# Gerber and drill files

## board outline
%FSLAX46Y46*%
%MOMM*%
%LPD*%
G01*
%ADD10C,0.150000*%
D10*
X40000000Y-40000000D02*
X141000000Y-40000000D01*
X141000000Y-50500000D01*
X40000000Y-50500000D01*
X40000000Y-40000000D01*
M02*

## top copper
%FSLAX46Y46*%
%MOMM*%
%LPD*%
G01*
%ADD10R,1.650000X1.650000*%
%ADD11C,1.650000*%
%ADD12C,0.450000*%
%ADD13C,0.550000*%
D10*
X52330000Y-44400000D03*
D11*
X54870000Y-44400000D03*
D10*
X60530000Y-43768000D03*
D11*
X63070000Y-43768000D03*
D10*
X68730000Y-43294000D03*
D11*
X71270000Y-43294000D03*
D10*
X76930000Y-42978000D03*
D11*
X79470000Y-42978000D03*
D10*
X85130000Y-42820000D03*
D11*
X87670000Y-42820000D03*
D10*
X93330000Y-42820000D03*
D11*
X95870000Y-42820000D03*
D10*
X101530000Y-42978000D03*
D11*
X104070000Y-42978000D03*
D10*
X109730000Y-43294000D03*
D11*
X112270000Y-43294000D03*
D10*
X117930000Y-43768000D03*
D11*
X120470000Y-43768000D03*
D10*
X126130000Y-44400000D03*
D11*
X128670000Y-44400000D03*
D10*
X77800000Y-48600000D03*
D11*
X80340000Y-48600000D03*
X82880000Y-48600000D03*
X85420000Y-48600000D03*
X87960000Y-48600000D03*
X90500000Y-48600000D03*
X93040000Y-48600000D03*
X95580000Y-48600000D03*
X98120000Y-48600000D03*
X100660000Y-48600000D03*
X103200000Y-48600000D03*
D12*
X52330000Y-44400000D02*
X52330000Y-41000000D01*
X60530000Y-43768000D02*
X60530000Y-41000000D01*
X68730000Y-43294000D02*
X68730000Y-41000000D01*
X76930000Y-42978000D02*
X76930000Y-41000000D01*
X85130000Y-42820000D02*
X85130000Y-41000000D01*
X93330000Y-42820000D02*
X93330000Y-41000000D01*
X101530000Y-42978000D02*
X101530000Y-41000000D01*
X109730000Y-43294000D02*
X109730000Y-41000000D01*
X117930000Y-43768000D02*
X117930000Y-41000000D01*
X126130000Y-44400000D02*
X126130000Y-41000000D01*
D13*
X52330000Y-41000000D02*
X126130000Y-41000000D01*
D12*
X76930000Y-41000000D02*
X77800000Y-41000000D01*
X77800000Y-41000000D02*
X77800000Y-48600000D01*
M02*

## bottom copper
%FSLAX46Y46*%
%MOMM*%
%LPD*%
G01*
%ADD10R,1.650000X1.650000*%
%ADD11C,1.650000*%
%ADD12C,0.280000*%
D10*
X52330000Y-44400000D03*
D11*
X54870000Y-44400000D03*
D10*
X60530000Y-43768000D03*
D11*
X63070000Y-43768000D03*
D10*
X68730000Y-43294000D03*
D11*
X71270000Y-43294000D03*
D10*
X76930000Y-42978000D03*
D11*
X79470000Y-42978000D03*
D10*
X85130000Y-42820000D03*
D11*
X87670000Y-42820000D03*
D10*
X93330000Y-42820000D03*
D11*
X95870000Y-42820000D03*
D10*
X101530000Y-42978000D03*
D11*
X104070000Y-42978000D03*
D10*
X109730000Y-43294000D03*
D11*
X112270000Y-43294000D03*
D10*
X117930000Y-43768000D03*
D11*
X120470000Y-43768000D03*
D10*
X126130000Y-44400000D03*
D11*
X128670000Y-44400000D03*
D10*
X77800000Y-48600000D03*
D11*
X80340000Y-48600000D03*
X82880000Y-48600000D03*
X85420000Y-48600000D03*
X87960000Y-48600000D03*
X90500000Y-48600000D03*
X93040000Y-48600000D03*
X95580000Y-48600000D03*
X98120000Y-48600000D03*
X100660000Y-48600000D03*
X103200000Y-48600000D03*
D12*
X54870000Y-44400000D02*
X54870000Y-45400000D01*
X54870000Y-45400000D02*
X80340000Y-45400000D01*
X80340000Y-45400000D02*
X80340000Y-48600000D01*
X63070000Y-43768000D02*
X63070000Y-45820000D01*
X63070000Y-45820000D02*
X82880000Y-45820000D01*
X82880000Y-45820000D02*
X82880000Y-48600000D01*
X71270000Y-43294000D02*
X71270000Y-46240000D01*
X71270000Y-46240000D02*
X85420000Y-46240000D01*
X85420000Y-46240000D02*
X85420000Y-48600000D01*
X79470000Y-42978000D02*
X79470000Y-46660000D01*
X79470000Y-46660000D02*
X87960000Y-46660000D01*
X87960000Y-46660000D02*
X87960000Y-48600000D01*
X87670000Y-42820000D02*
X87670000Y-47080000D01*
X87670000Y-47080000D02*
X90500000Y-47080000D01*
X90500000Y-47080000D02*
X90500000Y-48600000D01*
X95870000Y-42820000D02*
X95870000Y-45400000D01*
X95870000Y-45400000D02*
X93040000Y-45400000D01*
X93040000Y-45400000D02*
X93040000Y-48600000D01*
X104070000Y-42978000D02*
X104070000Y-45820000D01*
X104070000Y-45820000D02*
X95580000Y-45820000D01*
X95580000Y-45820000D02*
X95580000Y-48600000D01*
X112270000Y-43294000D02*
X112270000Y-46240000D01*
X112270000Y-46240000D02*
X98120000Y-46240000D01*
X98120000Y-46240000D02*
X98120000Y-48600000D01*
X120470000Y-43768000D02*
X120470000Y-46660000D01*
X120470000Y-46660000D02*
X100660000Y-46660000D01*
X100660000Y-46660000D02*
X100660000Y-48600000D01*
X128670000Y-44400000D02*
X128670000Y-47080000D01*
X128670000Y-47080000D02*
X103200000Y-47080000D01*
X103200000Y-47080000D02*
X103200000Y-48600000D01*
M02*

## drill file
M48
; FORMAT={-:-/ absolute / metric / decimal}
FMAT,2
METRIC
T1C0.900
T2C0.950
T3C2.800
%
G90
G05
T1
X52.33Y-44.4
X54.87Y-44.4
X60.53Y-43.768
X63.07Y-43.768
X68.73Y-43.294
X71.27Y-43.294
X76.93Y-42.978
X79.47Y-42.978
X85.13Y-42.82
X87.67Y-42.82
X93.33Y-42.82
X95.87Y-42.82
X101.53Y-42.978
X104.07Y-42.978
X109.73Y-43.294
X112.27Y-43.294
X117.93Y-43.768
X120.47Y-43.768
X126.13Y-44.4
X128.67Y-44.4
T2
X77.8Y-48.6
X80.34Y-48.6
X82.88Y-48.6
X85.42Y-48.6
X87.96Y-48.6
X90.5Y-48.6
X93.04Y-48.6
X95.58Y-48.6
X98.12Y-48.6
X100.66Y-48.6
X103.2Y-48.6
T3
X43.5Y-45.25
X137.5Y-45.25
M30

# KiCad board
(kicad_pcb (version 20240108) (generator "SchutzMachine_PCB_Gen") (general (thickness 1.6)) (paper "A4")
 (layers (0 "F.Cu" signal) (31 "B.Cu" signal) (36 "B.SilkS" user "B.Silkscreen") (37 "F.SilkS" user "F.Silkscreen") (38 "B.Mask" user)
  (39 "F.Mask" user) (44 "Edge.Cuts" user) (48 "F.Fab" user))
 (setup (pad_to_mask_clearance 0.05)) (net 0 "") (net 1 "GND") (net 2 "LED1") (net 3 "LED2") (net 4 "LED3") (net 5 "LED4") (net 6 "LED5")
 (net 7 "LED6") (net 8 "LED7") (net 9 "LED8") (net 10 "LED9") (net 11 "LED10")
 (gr_rect (start 40.0 40.0) (end 141.0 50.5) (stroke (width 0.15) (type solid)) (fill none) (layer "Edge.Cuts"))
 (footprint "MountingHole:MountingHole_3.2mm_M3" (layer "F.Cu") (at 43.5 45.25)
  (pad "" np_thru_hole circle (at 0 0) (size 2.8 2.8) (drill 2.8) (layers "*.Cu" "*.Mask")))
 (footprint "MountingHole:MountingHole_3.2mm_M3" (layer "F.Cu") (at 137.5 45.25)
  (pad "" np_thru_hole circle (at 0 0) (size 2.8 2.8) (drill 2.8) (layers "*.Cu" "*.Mask")))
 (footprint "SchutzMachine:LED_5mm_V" (layer "F.Cu") (at 53.6 44.4 0)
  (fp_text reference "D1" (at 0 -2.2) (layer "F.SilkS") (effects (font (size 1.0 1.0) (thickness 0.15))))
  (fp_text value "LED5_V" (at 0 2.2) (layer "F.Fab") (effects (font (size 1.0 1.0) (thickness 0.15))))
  (pad "1" thru_hole rect (at -1.27 0.0) (size 1.65 1.65) (drill 0.9) (layers "*.Cu" "*.Mask") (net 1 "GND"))
  (pad "2" thru_hole circle (at 1.27 0.0) (size 1.65 1.65) (drill 0.9) (layers "*.Cu" "*.Mask") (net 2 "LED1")))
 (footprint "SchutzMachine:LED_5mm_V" (layer "F.Cu") (at 61.8 43.768 0)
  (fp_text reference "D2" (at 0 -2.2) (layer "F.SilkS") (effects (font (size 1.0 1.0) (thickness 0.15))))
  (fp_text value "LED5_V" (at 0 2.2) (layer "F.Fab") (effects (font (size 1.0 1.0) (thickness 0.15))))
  (pad "1" thru_hole rect (at -1.27 0.0) (size 1.65 1.65) (drill 0.9) (layers "*.Cu" "*.Mask") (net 1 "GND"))
  (pad "2" thru_hole circle (at 1.27 0.0) (size 1.65 1.65) (drill 0.9) (layers "*.Cu" "*.Mask") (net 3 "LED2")))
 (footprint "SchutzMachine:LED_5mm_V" (layer "F.Cu") (at 70.0 43.294 0)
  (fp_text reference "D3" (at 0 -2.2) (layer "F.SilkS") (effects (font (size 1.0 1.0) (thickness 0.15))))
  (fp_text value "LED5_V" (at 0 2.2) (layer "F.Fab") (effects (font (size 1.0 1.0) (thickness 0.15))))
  (pad "1" thru_hole rect (at -1.27 0.0) (size 1.65 1.65) (drill 0.9) (layers "*.Cu" "*.Mask") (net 1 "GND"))
  (pad "2" thru_hole circle (at 1.27 0.0) (size 1.65 1.65) (drill 0.9) (layers "*.Cu" "*.Mask") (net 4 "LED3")))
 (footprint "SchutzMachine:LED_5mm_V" (layer "F.Cu") (at 78.2 42.978 0)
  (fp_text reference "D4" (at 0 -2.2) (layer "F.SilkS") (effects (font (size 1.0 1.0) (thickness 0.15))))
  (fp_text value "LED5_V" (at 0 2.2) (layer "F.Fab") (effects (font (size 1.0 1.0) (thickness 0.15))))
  (pad "1" thru_hole rect (at -1.27 0.0) (size 1.65 1.65) (drill 0.9) (layers "*.Cu" "*.Mask") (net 1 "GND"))
  (pad "2" thru_hole circle (at 1.27 0.0) (size 1.65 1.65) (drill 0.9) (layers "*.Cu" "*.Mask") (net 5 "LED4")))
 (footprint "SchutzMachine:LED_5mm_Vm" (layer "F.Cu") (at 86.4 42.82 0)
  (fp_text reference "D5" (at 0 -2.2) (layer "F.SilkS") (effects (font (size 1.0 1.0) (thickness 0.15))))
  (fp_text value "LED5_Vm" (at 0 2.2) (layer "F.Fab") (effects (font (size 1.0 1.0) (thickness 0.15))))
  (pad "1" thru_hole rect (at -1.27 0.0) (size 1.65 1.65) (drill 0.9) (layers "*.Cu" "*.Mask") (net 1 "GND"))
  (pad "2" thru_hole circle (at 1.27 0.0) (size 1.65 1.65) (drill 0.9) (layers "*.Cu" "*.Mask") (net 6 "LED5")))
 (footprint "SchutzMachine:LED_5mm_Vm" (layer "F.Cu") (at 94.6 42.82 0)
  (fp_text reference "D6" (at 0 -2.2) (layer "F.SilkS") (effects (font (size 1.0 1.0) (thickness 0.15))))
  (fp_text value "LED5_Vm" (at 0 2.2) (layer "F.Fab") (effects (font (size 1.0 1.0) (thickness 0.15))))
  (pad "1" thru_hole rect (at -1.27 0.0) (size 1.65 1.65) (drill 0.9) (layers "*.Cu" "*.Mask") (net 1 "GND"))
  (pad "2" thru_hole circle (at 1.27 0.0) (size 1.65 1.65) (drill 0.9) (layers "*.Cu" "*.Mask") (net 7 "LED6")))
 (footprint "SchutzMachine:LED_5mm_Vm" (layer "F.Cu") (at 102.8 42.978 0)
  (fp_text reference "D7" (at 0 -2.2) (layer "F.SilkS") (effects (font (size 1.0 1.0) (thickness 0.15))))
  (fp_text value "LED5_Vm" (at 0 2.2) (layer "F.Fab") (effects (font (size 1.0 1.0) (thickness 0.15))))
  (pad "1" thru_hole rect (at -1.27 0.0) (size 1.65 1.65) (drill 0.9) (layers "*.Cu" "*.Mask") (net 1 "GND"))
  (pad "2" thru_hole circle (at 1.27 0.0) (size 1.65 1.65) (drill 0.9) (layers "*.Cu" "*.Mask") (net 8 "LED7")))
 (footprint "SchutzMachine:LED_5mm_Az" (layer "F.Cu") (at 111.0 43.294 0)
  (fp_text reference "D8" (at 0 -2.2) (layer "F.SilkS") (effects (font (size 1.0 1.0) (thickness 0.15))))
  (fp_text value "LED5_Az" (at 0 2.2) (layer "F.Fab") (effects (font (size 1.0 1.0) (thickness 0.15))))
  (pad "1" thru_hole rect (at -1.27 0.0) (size 1.65 1.65) (drill 0.9) (layers "*.Cu" "*.Mask") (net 1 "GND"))
  (pad "2" thru_hole circle (at 1.27 0.0) (size 1.65 1.65) (drill 0.9) (layers "*.Cu" "*.Mask") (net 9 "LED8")))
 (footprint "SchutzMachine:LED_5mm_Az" (layer "F.Cu") (at 119.2 43.768 0)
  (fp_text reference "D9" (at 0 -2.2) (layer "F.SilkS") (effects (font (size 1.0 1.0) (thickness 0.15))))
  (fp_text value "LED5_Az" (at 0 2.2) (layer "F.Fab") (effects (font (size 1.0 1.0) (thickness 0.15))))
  (pad "1" thru_hole rect (at -1.27 0.0) (size 1.65 1.65) (drill 0.9) (layers "*.Cu" "*.Mask") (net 1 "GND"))
  (pad "2" thru_hole circle (at 1.27 0.0) (size 1.65 1.65) (drill 0.9) (layers "*.Cu" "*.Mask") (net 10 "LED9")))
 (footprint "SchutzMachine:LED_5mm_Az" (layer "F.Cu") (at 127.4 44.4 0)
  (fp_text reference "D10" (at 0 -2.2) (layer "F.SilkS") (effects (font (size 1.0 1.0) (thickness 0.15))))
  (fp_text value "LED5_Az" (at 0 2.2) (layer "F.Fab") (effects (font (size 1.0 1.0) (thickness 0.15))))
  (pad "1" thru_hole rect (at -1.27 0.0) (size 1.65 1.65) (drill 0.9) (layers "*.Cu" "*.Mask") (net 1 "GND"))
  (pad "2" thru_hole circle (at 1.27 0.0) (size 1.65 1.65) (drill 0.9) (layers "*.Cu" "*.Mask") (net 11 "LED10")))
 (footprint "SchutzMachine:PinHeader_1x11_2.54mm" (layer "F.Cu") (at 90.5 48.6 0)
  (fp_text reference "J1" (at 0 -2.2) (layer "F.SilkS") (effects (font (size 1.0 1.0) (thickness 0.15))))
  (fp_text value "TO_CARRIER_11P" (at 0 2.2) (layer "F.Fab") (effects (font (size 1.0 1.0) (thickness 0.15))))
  (pad "1" thru_hole rect (at -12.7 0.0) (size 1.65 1.65) (drill 0.95) (layers "*.Cu" "*.Mask") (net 1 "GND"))
  (pad "2" thru_hole circle (at -10.16 0.0) (size 1.65 1.65) (drill 0.95) (layers "*.Cu" "*.Mask") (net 2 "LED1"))
  (pad "3" thru_hole circle (at -7.62 0.0) (size 1.65 1.65) (drill 0.95) (layers "*.Cu" "*.Mask") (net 3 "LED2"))
  (pad "4" thru_hole circle (at -5.08 0.0) (size 1.65 1.65) (drill 0.95) (layers "*.Cu" "*.Mask") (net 4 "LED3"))
  (pad "5" thru_hole circle (at -2.54 0.0) (size 1.65 1.65) (drill 0.95) (layers "*.Cu" "*.Mask") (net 5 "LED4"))
  (pad "6" thru_hole circle (at 0.0 0.0) (size 1.65 1.65) (drill 0.95) (layers "*.Cu" "*.Mask") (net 6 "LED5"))
  (pad "7" thru_hole circle (at 2.54 0.0) (size 1.65 1.65) (drill 0.95) (layers "*.Cu" "*.Mask") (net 7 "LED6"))
  (pad "8" thru_hole circle (at 5.08 0.0) (size 1.65 1.65) (drill 0.95) (layers "*.Cu" "*.Mask") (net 8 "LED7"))
  (pad "9" thru_hole circle (at 7.62 0.0) (size 1.65 1.65) (drill 0.95) (layers "*.Cu" "*.Mask") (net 9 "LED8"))
  (pad "10" thru_hole circle (at 10.16 0.0) (size 1.65 1.65) (drill 0.95) (layers "*.Cu" "*.Mask") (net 10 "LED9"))
  (pad "11" thru_hole circle (at 12.7 0.0) (size 1.65 1.65) (drill 0.95) (layers "*.Cu" "*.Mask") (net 11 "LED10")))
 (segment (start 52.33 44.4) (end 52.33 41.0) (width 0.45) (layer "F.Cu") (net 1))
 (segment (start 60.53 43.768) (end 60.53 41.0) (width 0.45) (layer "F.Cu") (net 1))
 (segment (start 68.73 43.294) (end 68.73 41.0) (width 0.45) (layer "F.Cu") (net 1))
 (segment (start 76.93 42.978) (end 76.93 41.0) (width 0.45) (layer "F.Cu") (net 1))
 (segment (start 85.13 42.82) (end 85.13 41.0) (width 0.45) (layer "F.Cu") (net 1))
 (segment (start 93.33 42.82) (end 93.33 41.0) (width 0.45) (layer "F.Cu") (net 1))
 (segment (start 101.53 42.978) (end 101.53 41.0) (width 0.45) (layer "F.Cu") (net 1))
 (segment (start 109.73 43.294) (end 109.73 41.0) (width 0.45) (layer "F.Cu") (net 1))
 (segment (start 117.93 43.768) (end 117.93 41.0) (width 0.45) (layer "F.Cu") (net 1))
 (segment (start 126.13 44.4) (end 126.13 41.0) (width 0.45) (layer "F.Cu") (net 1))
 (segment (start 52.33 41.0) (end 126.13 41.0) (width 0.55) (layer "F.Cu") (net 1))
 (segment (start 76.93 41.0) (end 77.8 41.0) (width 0.45) (layer "F.Cu") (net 1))
 (segment (start 77.8 41.0) (end 77.8 48.6) (width 0.45) (layer "F.Cu") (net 1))
 (segment (start 54.87 44.4) (end 54.87 45.4) (width 0.28) (layer "B.Cu") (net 2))
 (segment (start 54.87 45.4) (end 80.34 45.4) (width 0.28) (layer "B.Cu") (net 2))
 (segment (start 80.34 45.4) (end 80.34 48.6) (width 0.28) (layer "B.Cu") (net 2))
 (segment (start 63.07 43.768) (end 63.07 45.82) (width 0.28) (layer "B.Cu") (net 3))
 (segment (start 63.07 45.82) (end 82.88 45.82) (width 0.28) (layer "B.Cu") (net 3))
 (segment (start 82.88 45.82) (end 82.88 48.6) (width 0.28) (layer "B.Cu") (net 3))
 (segment (start 71.27 43.294) (end 71.27 46.24) (width 0.28) (layer "B.Cu") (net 4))
 (segment (start 71.27 46.24) (end 85.42 46.24) (width 0.28) (layer "B.Cu") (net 4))
 (segment (start 85.42 46.24) (end 85.42 48.6) (width 0.28) (layer "B.Cu") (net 4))
 (segment (start 79.47 42.978) (end 79.47 46.66) (width 0.28) (layer "B.Cu") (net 5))
 (segment (start 79.47 46.66) (end 87.96 46.66) (width 0.28) (layer "B.Cu") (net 5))
 (segment (start 87.96 46.66) (end 87.96 48.6) (width 0.28) (layer "B.Cu") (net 5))
 (segment (start 87.67 42.82) (end 87.67 47.08) (width 0.28) (layer "B.Cu") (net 6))
 (segment (start 87.67 47.08) (end 90.5 47.08) (width 0.28) (layer "B.Cu") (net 6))
 (segment (start 90.5 47.08) (end 90.5 48.6) (width 0.28) (layer "B.Cu") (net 6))
 (segment (start 95.87 42.82) (end 95.87 45.4) (width 0.28) (layer "B.Cu") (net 7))
 (segment (start 95.87 45.4) (end 93.04 45.4) (width 0.28) (layer "B.Cu") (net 7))
 (segment (start 93.04 45.4) (end 93.04 48.6) (width 0.28) (layer "B.Cu") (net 7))
 (segment (start 104.07 42.978) (end 104.07 45.82) (width 0.28) (layer "B.Cu") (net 8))
 (segment (start 104.07 45.82) (end 95.58 45.82) (width 0.28) (layer "B.Cu") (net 8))
 (segment (start 95.58 45.82) (end 95.58 48.6) (width 0.28) (layer "B.Cu") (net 8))
 (segment (start 112.27 43.294) (end 112.27 46.24) (width 0.28) (layer "B.Cu") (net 9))
 (segment (start 112.27 46.24) (end 98.12 46.24) (width 0.28) (layer "B.Cu") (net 9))
 (segment (start 98.12 46.24) (end 98.12 48.6) (width 0.28) (layer "B.Cu") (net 9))
 (segment (start 120.47 43.768) (end 120.47 46.66) (width 0.28) (layer "B.Cu") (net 10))
 (segment (start 120.47 46.66) (end 100.66 46.66) (width 0.28) (layer "B.Cu") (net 10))
 (segment (start 100.66 46.66) (end 100.66 48.6) (width 0.28) (layer "B.Cu") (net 10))
 (segment (start 128.67 44.4) (end 128.67 47.08) (width 0.28) (layer "B.Cu") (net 11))
 (segment (start 128.67 47.08) (end 103.2 47.08) (width 0.28) (layer "B.Cu") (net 11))
 (segment (start 103.2 47.08) (end 103.2 48.6) (width 0.28) (layer "B.Cu") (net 11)))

